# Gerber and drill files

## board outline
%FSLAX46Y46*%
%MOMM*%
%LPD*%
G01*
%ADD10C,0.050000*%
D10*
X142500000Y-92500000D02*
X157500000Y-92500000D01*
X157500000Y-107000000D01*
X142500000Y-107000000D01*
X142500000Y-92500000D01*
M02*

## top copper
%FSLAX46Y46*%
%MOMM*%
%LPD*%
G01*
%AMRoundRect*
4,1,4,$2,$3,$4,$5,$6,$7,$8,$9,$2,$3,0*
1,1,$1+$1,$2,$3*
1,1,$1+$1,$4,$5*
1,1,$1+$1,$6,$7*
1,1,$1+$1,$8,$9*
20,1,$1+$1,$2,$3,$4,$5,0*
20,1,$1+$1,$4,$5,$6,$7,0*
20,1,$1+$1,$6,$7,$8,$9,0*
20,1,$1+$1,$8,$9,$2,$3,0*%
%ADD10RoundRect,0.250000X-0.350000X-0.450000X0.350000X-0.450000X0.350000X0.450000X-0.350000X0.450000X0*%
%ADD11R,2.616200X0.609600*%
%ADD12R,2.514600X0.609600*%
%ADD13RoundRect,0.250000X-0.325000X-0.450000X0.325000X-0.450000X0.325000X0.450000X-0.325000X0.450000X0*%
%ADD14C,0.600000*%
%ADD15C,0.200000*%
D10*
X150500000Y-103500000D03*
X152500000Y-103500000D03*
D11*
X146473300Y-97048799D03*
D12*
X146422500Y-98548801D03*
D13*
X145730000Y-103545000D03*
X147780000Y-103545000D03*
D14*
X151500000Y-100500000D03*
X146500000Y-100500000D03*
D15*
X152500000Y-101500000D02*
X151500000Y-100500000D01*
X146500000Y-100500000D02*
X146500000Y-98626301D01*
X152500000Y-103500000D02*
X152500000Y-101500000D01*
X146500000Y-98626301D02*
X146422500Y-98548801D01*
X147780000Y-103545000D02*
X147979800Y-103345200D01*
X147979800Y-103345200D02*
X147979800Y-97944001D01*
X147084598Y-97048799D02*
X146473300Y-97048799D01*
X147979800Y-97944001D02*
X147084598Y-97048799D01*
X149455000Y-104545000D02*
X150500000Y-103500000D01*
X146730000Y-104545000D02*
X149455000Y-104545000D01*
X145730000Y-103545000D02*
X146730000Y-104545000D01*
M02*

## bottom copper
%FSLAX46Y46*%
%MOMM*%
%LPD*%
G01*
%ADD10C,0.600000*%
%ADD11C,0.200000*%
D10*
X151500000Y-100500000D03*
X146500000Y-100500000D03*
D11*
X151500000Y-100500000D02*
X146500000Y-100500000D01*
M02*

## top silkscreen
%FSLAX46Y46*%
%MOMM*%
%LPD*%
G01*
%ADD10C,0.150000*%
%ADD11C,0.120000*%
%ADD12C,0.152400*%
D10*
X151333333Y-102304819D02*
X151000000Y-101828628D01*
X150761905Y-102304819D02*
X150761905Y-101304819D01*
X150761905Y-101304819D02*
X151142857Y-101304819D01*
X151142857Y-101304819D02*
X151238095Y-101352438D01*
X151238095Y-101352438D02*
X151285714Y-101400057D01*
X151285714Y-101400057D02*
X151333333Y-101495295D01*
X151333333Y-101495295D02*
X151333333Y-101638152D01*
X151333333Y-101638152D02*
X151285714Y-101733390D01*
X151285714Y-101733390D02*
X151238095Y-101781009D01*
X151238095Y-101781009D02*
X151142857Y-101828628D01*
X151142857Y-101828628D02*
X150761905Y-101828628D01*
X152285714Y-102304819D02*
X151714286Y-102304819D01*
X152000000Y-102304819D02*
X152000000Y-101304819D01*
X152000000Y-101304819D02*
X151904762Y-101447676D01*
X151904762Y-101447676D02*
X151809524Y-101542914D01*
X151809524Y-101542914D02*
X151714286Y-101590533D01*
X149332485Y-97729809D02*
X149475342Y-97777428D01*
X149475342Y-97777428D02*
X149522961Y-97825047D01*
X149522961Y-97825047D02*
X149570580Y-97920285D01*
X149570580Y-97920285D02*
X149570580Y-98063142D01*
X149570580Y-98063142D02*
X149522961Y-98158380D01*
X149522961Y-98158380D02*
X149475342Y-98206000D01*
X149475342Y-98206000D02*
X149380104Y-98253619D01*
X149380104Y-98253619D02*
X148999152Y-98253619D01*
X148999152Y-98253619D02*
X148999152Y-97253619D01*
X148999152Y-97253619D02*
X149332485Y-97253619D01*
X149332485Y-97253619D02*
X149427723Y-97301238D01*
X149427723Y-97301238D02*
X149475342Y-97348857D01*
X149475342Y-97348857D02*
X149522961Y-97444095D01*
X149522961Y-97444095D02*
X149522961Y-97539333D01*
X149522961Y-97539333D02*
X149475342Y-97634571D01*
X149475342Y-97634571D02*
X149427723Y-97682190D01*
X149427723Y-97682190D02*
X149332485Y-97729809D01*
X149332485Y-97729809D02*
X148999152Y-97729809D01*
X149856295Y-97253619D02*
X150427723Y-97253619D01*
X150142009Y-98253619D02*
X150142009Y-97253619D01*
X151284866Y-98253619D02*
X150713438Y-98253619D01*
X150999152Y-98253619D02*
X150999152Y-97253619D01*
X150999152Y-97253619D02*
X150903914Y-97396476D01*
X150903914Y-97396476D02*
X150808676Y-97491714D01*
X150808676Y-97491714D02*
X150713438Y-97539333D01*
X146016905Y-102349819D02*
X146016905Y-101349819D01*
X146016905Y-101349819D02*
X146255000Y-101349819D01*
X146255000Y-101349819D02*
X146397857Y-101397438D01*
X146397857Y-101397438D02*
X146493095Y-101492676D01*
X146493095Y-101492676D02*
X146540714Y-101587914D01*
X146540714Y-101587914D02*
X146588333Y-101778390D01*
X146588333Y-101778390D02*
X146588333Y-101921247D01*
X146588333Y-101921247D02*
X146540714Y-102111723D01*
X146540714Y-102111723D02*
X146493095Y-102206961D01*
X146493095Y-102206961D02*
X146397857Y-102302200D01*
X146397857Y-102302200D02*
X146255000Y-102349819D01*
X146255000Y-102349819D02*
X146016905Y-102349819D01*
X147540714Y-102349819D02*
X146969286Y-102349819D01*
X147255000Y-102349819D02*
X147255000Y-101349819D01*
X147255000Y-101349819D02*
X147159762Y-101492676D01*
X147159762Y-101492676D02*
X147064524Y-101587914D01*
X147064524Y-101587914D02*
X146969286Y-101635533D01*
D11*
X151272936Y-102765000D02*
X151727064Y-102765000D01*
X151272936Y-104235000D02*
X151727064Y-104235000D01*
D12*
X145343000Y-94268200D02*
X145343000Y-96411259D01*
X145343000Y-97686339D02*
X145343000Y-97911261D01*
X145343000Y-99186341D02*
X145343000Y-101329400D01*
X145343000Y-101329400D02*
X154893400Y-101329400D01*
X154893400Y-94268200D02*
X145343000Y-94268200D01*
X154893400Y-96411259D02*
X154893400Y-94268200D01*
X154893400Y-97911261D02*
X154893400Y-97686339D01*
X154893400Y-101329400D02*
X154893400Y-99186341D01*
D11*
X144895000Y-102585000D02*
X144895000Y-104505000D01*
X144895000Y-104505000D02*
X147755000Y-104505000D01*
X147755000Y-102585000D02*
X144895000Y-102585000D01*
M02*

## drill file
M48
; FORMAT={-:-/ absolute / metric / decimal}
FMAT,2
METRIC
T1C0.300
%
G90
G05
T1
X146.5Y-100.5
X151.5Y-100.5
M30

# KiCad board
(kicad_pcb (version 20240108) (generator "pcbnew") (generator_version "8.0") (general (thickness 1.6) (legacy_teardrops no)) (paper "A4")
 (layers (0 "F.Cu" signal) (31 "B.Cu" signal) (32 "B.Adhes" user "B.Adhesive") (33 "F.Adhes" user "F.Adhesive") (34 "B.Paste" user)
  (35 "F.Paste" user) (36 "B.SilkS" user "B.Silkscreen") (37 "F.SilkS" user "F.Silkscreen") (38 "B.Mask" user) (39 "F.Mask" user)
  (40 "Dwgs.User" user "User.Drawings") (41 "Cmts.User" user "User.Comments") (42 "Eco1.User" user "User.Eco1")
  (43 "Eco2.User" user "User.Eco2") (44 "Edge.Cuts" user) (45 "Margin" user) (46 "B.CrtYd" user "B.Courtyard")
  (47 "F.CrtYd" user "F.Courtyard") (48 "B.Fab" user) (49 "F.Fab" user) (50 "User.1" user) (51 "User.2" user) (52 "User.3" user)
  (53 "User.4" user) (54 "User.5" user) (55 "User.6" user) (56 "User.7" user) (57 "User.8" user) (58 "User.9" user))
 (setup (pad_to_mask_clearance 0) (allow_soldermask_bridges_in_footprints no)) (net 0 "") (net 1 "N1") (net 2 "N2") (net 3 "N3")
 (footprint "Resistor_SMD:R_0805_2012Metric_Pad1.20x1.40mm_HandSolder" (layer "F.Cu") (at 151.5 103.5)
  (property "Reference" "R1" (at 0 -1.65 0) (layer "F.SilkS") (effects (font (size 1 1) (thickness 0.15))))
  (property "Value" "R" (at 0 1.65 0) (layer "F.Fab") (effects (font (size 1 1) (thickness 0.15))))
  (fp_line (start -0.227064 -0.735) (end 0.227064 -0.735) (stroke (width 0.12) (type solid)) (layer "F.SilkS"))
  (fp_line (start -0.227064 0.735) (end 0.227064 0.735) (stroke (width 0.12) (type solid)) (layer "F.SilkS"))
  (pad "1" smd roundrect (at -1 0) (size 1.2 1.4) (layers "F.Cu" "F.Paste" "F.Mask") (roundrect_rratio 0.208333) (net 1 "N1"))
  (pad "2" smd roundrect (at 1 0) (size 1.2 1.4) (layers "F.Cu" "F.Paste" "F.Mask") (roundrect_rratio 0.208333) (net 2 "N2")))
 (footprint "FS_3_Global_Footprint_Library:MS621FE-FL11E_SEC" (layer "F.Cu") (at 150.1182 97.7988)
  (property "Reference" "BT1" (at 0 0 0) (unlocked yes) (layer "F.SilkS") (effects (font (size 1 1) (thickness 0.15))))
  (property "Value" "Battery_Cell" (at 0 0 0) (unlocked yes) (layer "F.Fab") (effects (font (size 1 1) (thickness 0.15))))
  (fp_line (start -4.7752 -3.5306) (end -4.7752 -1.387541) (stroke (width 0.1524) (type solid)) (layer "F.SilkS"))
  (fp_line (start -4.7752 -0.112461) (end -4.7752 0.112461) (stroke (width 0.1524) (type solid)) (layer "F.SilkS"))
  (fp_line (start -4.7752 1.387541) (end -4.7752 3.5306) (stroke (width 0.1524) (type solid)) (layer "F.SilkS"))
  (fp_line (start -4.7752 3.5306) (end 4.7752 3.5306) (stroke (width 0.1524) (type solid)) (layer "F.SilkS"))
  (fp_line (start 4.7752 -3.5306) (end -4.7752 -3.5306) (stroke (width 0.1524) (type solid)) (layer "F.SilkS"))
  (fp_line (start 4.7752 -1.387541) (end 4.7752 -3.5306) (stroke (width 0.1524) (type solid)) (layer "F.SilkS"))
  (fp_line (start 4.7752 0.112461) (end 4.7752 -0.112461) (stroke (width 0.1524) (type solid)) (layer "F.SilkS"))
  (fp_line (start 4.7752 3.5306) (end 4.7752 1.387541) (stroke (width 0.1524) (type solid)) (layer "F.SilkS"))
  (pad "1" smd rect (at -3.6449 -0.750001) (size 2.6162 0.6096) (layers "F.Cu" "F.Paste" "F.Mask") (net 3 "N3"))
  (pad "2" smd rect (at -3.6957 0.750001) (size 2.5146 0.6096) (layers "F.Cu" "F.Paste" "F.Mask") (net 2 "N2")))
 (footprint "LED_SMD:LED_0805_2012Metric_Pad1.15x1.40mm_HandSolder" (layer "F.Cu") (at 146.755 103.545)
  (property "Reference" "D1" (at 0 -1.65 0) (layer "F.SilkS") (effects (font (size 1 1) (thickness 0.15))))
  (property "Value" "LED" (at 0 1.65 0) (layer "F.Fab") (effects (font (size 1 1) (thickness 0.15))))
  (fp_line (start -1.86 -0.96) (end -1.86 0.96) (stroke (width 0.12) (type solid)) (layer "F.SilkS"))
  (fp_line (start -1.86 0.96) (end 1 0.96) (stroke (width 0.12) (type solid)) (layer "F.SilkS"))
  (fp_line (start 1 -0.96) (end -1.86 -0.96) (stroke (width 0.12) (type solid)) (layer "F.SilkS"))
  (pad "1" smd roundrect (at -1.025 0) (size 1.15 1.4) (layers "F.Cu" "F.Paste" "F.Mask") (roundrect_rratio 0.217391) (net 1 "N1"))
  (pad "2" smd roundrect (at 1.025 0) (size 1.15 1.4) (layers "F.Cu" "F.Paste" "F.Mask") (roundrect_rratio 0.217391) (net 3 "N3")))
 (gr_rect (start 142.5 92.5) (end 157.5 107) (stroke (width 0.05) (type default)) (fill none) (layer "Edge.Cuts"))
 (segment (start 152.5 101.5) (end 151.5 100.5) (width 0.2) (layer "F.Cu") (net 2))
 (segment (start 146.5 100.5) (end 146.5 98.626301) (width 0.2) (layer "F.Cu") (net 2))
 (segment (start 152.5 103.5) (end 152.5 101.5) (width 0.2) (layer "F.Cu") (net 2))
 (segment (start 146.5 98.626301) (end 146.4225 98.548801) (width 0.2) (layer "F.Cu") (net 2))
 (via (at 151.5 100.5) (size 0.6) (drill 0.3) (layers "F.Cu" "B.Cu") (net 2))
 (via (at 146.5 100.5) (size 0.6) (drill 0.3) (layers "F.Cu" "B.Cu") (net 2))
 (segment (start 151.5 100.5) (end 146.5 100.5) (width 0.2) (layer "B.Cu") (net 2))
 (segment (start 147.78 103.545) (end 147.9798 103.3452) (width 0.2) (layer "F.Cu") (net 3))
 (segment (start 147.9798 103.3452) (end 147.9798 97.944001) (width 0.2) (layer "F.Cu") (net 3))
 (segment (start 147.084598 97.048799) (end 146.4733 97.048799) (width 0.2) (layer "F.Cu") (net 3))
 (segment (start 147.9798 97.944001) (end 147.084598 97.048799) (width 0.2) (layer "F.Cu") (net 3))
 (segment (start 149.455 104.545) (end 150.5 103.5) (width 0.2) (layer "F.Cu") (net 1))
 (segment (start 146.73 104.545) (end 149.455 104.545) (width 0.2) (layer "F.Cu") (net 1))
 (segment (start 145.73 103.545) (end 146.73 104.545) (width 0.2) (layer "F.Cu") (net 1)))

